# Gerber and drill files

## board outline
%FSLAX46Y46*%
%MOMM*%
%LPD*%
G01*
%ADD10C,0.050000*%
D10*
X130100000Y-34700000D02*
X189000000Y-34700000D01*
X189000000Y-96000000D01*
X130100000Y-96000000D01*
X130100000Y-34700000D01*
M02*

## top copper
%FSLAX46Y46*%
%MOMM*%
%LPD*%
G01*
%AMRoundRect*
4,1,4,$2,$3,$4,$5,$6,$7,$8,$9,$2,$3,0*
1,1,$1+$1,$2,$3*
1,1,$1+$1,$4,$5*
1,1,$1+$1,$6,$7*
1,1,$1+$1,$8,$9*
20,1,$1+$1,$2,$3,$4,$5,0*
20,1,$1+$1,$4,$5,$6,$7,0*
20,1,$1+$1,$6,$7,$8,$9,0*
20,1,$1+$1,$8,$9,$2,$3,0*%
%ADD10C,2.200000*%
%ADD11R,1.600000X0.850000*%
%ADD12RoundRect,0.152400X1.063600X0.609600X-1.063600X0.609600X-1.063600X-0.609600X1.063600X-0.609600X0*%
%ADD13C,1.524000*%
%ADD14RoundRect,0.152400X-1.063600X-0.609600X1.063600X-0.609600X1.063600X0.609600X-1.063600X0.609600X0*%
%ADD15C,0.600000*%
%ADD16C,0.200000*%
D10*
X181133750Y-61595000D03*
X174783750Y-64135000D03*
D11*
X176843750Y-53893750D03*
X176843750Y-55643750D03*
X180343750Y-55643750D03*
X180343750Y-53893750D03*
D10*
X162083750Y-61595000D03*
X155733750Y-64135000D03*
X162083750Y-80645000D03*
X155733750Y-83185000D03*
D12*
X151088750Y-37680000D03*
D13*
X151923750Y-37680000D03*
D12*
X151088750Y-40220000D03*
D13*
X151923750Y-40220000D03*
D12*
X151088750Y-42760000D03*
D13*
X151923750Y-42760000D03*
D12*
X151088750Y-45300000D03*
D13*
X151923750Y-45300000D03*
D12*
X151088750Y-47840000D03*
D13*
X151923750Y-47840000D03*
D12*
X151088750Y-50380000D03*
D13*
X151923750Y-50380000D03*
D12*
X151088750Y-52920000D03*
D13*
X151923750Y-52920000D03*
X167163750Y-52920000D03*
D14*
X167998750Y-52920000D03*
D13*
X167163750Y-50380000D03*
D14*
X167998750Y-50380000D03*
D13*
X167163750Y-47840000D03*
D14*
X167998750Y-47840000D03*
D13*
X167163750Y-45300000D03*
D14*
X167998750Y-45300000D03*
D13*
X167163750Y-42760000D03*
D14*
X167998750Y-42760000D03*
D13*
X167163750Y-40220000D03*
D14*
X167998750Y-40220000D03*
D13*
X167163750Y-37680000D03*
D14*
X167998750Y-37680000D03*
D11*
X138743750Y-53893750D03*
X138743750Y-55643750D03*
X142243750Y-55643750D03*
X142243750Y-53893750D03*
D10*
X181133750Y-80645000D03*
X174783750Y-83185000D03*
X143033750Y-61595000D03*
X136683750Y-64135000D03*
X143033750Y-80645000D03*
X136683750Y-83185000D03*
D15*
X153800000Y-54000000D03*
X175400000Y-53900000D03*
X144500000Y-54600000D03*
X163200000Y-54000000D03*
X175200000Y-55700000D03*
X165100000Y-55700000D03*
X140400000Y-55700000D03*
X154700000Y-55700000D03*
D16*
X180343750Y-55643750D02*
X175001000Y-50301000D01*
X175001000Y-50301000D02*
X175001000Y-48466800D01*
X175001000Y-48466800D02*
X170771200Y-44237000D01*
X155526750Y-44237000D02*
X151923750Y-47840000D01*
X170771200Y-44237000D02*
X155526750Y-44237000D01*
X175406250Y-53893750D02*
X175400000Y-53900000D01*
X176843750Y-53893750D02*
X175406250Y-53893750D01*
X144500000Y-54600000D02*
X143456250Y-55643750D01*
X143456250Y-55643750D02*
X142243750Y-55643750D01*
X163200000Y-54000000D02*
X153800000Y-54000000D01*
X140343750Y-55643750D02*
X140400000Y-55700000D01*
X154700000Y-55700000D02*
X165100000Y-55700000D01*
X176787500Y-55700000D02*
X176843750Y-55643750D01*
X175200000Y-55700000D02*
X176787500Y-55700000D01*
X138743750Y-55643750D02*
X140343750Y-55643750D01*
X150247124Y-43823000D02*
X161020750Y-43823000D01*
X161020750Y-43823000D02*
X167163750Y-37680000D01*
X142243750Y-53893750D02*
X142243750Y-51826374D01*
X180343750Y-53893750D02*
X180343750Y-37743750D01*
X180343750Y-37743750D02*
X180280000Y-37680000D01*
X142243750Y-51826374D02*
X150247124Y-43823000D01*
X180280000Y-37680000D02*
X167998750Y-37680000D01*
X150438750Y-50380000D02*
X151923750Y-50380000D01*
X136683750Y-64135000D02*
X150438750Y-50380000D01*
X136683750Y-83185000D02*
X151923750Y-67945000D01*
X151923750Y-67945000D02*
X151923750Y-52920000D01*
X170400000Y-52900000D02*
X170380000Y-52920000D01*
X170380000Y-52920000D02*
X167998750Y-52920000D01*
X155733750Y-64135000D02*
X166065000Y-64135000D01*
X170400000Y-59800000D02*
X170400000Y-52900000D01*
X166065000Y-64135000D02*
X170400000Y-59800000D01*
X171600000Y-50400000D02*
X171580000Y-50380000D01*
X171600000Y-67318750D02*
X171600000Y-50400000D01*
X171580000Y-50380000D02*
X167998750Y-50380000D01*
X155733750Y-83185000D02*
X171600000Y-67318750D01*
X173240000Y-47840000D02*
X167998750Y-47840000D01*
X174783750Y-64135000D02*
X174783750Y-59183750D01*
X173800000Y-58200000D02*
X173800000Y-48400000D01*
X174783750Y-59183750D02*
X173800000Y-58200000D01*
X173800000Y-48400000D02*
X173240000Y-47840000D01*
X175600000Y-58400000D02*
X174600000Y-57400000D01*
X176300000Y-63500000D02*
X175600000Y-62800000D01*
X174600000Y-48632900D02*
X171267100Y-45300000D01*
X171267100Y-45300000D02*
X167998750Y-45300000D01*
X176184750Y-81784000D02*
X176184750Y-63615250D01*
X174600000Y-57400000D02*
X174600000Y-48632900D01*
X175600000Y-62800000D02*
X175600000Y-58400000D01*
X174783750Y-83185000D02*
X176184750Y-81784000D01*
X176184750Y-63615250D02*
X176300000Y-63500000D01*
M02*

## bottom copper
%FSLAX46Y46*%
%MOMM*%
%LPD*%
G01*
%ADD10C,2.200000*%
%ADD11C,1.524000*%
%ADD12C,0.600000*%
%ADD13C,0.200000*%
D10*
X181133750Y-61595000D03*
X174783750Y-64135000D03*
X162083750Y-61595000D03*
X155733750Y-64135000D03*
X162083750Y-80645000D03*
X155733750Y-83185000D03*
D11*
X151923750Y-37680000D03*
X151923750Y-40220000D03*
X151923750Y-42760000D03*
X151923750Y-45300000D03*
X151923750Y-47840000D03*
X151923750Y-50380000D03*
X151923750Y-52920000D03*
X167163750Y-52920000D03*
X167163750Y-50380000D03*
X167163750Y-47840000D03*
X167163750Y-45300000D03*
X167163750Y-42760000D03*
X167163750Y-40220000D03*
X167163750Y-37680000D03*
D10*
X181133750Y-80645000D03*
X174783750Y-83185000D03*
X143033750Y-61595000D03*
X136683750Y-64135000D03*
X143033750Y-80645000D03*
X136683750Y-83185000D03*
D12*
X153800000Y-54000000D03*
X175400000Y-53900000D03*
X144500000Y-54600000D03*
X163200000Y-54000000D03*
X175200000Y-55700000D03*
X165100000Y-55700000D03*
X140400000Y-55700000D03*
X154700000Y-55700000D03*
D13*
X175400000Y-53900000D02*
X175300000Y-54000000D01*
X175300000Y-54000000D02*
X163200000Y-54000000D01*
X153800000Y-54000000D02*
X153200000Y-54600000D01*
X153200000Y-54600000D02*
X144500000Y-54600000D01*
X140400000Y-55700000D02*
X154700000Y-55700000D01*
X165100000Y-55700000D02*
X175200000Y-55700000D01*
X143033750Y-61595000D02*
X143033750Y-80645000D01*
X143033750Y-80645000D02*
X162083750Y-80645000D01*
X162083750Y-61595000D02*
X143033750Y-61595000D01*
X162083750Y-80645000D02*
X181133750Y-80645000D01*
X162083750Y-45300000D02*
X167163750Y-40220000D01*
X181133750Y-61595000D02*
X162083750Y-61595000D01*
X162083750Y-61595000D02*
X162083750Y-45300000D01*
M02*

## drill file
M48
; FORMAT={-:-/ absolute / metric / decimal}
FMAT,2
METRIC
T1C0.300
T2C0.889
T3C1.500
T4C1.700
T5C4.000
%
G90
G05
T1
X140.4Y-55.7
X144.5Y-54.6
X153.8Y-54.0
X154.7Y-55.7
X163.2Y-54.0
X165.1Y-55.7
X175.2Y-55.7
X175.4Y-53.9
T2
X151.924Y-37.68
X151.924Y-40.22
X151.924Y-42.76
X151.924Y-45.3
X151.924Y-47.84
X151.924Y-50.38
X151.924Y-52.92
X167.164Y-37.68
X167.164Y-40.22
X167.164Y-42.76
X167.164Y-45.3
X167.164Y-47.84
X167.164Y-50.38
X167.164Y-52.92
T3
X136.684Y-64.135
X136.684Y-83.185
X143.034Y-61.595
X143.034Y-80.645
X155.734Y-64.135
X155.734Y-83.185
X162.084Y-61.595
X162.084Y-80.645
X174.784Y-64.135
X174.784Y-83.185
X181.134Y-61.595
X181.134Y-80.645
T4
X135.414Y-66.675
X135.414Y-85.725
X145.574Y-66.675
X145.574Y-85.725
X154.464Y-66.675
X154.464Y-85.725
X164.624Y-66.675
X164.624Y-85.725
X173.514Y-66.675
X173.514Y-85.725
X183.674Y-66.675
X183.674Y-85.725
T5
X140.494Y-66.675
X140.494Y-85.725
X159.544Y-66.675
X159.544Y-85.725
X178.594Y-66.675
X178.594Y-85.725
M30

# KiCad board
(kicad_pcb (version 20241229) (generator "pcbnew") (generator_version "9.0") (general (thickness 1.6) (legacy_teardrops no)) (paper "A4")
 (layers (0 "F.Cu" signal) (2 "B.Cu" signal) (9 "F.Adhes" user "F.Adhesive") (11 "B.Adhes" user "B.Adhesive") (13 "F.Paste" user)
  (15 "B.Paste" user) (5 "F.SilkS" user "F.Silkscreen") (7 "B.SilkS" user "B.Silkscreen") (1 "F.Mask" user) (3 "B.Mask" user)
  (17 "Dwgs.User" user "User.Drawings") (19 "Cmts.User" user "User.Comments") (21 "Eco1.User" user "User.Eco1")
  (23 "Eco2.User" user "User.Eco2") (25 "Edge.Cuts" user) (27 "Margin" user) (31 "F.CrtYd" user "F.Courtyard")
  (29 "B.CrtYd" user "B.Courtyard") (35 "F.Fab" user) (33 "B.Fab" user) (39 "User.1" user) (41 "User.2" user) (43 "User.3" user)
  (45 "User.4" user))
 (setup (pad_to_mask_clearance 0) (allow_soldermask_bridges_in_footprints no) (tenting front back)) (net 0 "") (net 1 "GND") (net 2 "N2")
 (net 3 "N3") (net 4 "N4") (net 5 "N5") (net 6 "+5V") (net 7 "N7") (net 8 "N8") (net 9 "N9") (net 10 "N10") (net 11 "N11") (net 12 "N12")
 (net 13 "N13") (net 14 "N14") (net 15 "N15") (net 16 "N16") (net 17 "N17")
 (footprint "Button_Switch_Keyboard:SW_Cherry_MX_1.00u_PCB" (layer "F.Cu") (at 181.13375 61.595)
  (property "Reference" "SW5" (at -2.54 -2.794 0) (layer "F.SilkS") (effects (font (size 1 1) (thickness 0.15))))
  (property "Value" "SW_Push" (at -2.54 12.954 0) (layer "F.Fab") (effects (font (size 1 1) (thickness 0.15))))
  (pad "" np_thru_hole circle (at -7.62 5.08) (size 1.7 1.7) (drill 1.7) (layers "*.Cu" "*.Mask"))
  (pad "" np_thru_hole circle (at -2.54 5.08) (size 4 4) (drill 4) (layers "*.Cu" "*.Mask"))
  (pad "" np_thru_hole circle (at 2.54 5.08) (size 1.7 1.7) (drill 1.7) (layers "*.Cu" "*.Mask"))
  (pad "1" thru_hole circle (at 0 0) (size 2.2 2.2) (drill 1.5) (layers "*.Cu" "*.Mask") (remove_unused_layers no) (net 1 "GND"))
  (pad "2" thru_hole circle (at -6.35 2.54) (size 2.2 2.2) (drill 1.5) (layers "*.Cu" "*.Mask") (remove_unused_layers no) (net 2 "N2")))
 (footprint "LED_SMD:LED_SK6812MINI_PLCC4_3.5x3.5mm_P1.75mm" (layer "F.Cu") (at 178.59375 54.76875)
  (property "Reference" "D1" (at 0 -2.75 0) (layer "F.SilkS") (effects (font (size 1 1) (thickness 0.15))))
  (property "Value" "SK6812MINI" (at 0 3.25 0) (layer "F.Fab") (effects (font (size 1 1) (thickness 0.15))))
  (pad "1" smd rect (at -1.75 -0.875) (size 1.6 0.85) (layers "F.Cu" "F.Mask" "F.Paste") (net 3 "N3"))
  (pad "2" smd rect (at -1.75 0.875) (size 1.6 0.85) (layers "F.Cu" "F.Mask" "F.Paste") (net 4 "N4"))
  (pad "3" smd rect (at 1.75 0.875) (size 1.6 0.85) (layers "F.Cu" "F.Mask" "F.Paste") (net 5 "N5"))
  (pad "4" smd rect (at 1.75 -0.875) (size 1.6 0.85) (layers "F.Cu" "F.Mask" "F.Paste") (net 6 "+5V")))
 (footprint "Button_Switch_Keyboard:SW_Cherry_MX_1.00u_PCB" (layer "F.Cu") (at 162.08375 61.595)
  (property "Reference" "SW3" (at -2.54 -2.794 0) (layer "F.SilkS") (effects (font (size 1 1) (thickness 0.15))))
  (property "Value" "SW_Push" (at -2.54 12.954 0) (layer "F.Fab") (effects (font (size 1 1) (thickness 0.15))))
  (pad "" np_thru_hole circle (at -7.62 5.08) (size 1.7 1.7) (drill 1.7) (layers "*.Cu" "*.Mask"))
  (pad "" np_thru_hole circle (at -2.54 5.08) (size 4 4) (drill 4) (layers "*.Cu" "*.Mask"))
  (pad "" np_thru_hole circle (at 2.54 5.08) (size 1.7 1.7) (drill 1.7) (layers "*.Cu" "*.Mask"))
  (pad "1" thru_hole circle (at 0 0) (size 2.2 2.2) (drill 1.5) (layers "*.Cu" "*.Mask") (remove_unused_layers no) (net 1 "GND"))
  (pad "2" thru_hole circle (at -6.35 2.54) (size 2.2 2.2) (drill 1.5) (layers "*.Cu" "*.Mask") (remove_unused_layers no) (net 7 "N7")))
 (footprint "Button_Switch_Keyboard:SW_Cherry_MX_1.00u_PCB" (layer "F.Cu") (at 162.08375 80.645)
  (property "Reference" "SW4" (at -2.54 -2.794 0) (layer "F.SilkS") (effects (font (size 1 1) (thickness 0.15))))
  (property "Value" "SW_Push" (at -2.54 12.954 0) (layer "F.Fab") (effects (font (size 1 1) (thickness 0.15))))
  (pad "" np_thru_hole circle (at -7.62 5.08) (size 1.7 1.7) (drill 1.7) (layers "*.Cu" "*.Mask"))
  (pad "" np_thru_hole circle (at -2.54 5.08) (size 4 4) (drill 4) (layers "*.Cu" "*.Mask"))
  (pad "" np_thru_hole circle (at 2.54 5.08) (size 1.7 1.7) (drill 1.7) (layers "*.Cu" "*.Mask"))
  (pad "1" thru_hole circle (at 0 0) (size 2.2 2.2) (drill 1.5) (layers "*.Cu" "*.Mask") (remove_unused_layers no) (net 1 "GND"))
  (pad "2" thru_hole circle (at -6.35 2.54) (size 2.2 2.2) (drill 1.5) (layers "*.Cu" "*.Mask") (remove_unused_layers no) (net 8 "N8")))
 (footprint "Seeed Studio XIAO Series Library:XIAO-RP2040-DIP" (layer "F.Cu") (at 159.54375 45.3)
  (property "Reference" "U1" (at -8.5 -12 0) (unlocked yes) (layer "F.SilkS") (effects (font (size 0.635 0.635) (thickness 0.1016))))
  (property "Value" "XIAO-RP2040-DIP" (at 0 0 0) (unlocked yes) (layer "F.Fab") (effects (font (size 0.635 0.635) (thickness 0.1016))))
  (pad "1" smd roundrect (at -8.455 -7.62 180) (size 2.432 1.524) (layers "F.Cu" "F.Mask") (roundrect_rratio 0.1) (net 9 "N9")
   (thermal_bridge_angle 45))
  (pad "1" thru_hole circle (at -7.62 -7.62 180) (size 1.524 1.524) (drill 0.889) (layers "*.Cu" "*.Mask") (remove_unused_layers no)
   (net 9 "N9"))
  (pad "2" smd roundrect (at -8.455 -5.08 180) (size 2.432 1.524) (layers "F.Cu" "F.Mask") (roundrect_rratio 0.1) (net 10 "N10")
   (thermal_bridge_angle 45))
  (pad "2" thru_hole circle (at -7.62 -5.08 180) (size 1.524 1.524) (drill 0.889) (layers "*.Cu" "*.Mask") (remove_unused_layers no)
   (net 10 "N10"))
  (pad "3" smd roundrect (at -8.455 -2.54 180) (size 2.432 1.524) (layers "F.Cu" "F.Mask") (roundrect_rratio 0.1) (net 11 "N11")
   (thermal_bridge_angle 45))
  (pad "3" thru_hole circle (at -7.62 -2.54 180) (size 1.524 1.524) (drill 0.889) (layers "*.Cu" "*.Mask") (remove_unused_layers no)
   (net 11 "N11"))
  (pad "4" smd roundrect (at -8.455 0 180) (size 2.432 1.524) (layers "F.Cu" "F.Mask") (roundrect_rratio 0.1) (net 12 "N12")
   (thermal_bridge_angle 45))
  (pad "4" thru_hole circle (at -7.62 0 180) (size 1.524 1.524) (drill 0.889) (layers "*.Cu" "*.Mask") (remove_unused_layers no)
   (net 12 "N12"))
  (pad "5" smd roundrect (at -8.455 2.54 180) (size 2.432 1.524) (layers "F.Cu" "F.Mask") (roundrect_rratio 0.1) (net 5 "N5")
   (thermal_bridge_angle 45))
  (pad "5" thru_hole circle (at -7.62 2.54 180) (size 1.524 1.524) (drill 0.889) (layers "*.Cu" "*.Mask") (remove_unused_layers no)
   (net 5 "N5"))
  (pad "6" smd roundrect (at -8.455 5.08 180) (size 2.432 1.524) (layers "F.Cu" "F.Mask") (roundrect_rratio 0.1) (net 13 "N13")
   (thermal_bridge_angle 45))
  (pad "6" thru_hole circle (at -7.62 5.08 180) (size 1.524 1.524) (drill 0.889) (layers "*.Cu" "*.Mask") (remove_unused_layers no)
   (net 13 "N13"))
  (pad "7" smd roundrect (at -8.455 7.62 180) (size 2.432 1.524) (layers "F.Cu" "F.Mask") (roundrect_rratio 0.1) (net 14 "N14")
   (thermal_bridge_angle 45))
  (pad "7" thru_hole circle (at -7.62 7.62 180) (size 1.524 1.524) (drill 0.889) (layers "*.Cu" "*.Mask") (remove_unused_layers no)
   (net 14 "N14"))
  (pad "8" thru_hole circle (at 7.62 7.62) (size 1.524 1.524) (drill 0.889) (layers "*.Cu" "*.Mask") (remove_unused_layers no) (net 7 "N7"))
  (pad "8" smd roundrect (at 8.455 7.62) (size 2.432 1.524) (layers "F.Cu" "F.Mask") (roundrect_rratio 0.1) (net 7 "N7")
   (thermal_bridge_angle 45))
  (pad "9" thru_hole circle (at 7.62 5.08) (size 1.524 1.524) (drill 0.889) (layers "*.Cu" "*.Mask") (remove_unused_layers no) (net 8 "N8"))
  (pad "9" smd roundrect (at 8.455 5.08) (size 2.432 1.524) (layers "F.Cu" "F.Mask") (roundrect_rratio 0.1) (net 8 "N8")
   (thermal_bridge_angle 45))
  (pad "10" thru_hole circle (at 7.62 2.54) (size 1.524 1.524) (drill 0.889) (layers "*.Cu" "*.Mask") (remove_unused_layers no) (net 2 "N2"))
  (pad "10" smd roundrect (at 8.455 2.54) (size 2.432 1.524) (layers "F.Cu" "F.Mask") (roundrect_rratio 0.1) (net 2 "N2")
   (thermal_bridge_angle 45))
  (pad "11" thru_hole circle (at 7.62 0) (size 1.524 1.524) (drill 0.889) (layers "*.Cu" "*.Mask") (remove_unused_layers no) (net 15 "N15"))
  (pad "11" smd roundrect (at 8.455 0) (size 2.432 1.524) (layers "F.Cu" "F.Mask") (roundrect_rratio 0.1) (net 15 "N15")
   (thermal_bridge_angle 45))
  (pad "12" thru_hole circle (at 7.62 -2.54) (size 1.524 1.524) (drill 0.889) (layers "*.Cu" "*.Mask") (remove_unused_layers no)
   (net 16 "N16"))
  (pad "12" smd roundrect (at 8.455 -2.54) (size 2.432 1.524) (layers "F.Cu" "F.Mask") (roundrect_rratio 0.1) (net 16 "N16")
   (thermal_bridge_angle 45))
  (pad "13" thru_hole circle (at 7.62 -5.08) (size 1.524 1.524) (drill 0.889) (layers "*.Cu" "*.Mask") (remove_unused_layers no)
   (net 1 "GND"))
  (pad "13" smd roundrect (at 8.455 -5.08) (size 2.432 1.524) (layers "F.Cu" "F.Mask") (roundrect_rratio 0.1) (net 1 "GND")
   (thermal_bridge_angle 45))
  (pad "14" thru_hole circle (at 7.62 -7.62) (size 1.524 1.524) (drill 0.889) (layers "*.Cu" "*.Mask") (remove_unused_layers no)
   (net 6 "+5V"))
  (pad "14" smd roundrect (at 8.455 -7.62) (size 2.432 1.524) (layers "F.Cu" "F.Mask") (roundrect_rratio 0.1) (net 6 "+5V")
   (thermal_bridge_angle 45)))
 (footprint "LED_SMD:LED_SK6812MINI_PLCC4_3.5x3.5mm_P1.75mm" (layer "F.Cu") (at 140.49375 54.76875)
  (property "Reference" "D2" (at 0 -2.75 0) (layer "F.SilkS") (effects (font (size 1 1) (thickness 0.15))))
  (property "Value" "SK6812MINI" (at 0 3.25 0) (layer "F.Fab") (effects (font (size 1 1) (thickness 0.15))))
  (pad "1" smd rect (at -1.75 -0.875) (size 1.6 0.85) (layers "F.Cu" "F.Mask" "F.Paste") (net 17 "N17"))
  (pad "2" smd rect (at -1.75 0.875) (size 1.6 0.85) (layers "F.Cu" "F.Mask" "F.Paste") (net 4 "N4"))
  (pad "3" smd rect (at 1.75 0.875) (size 1.6 0.85) (layers "F.Cu" "F.Mask" "F.Paste") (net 3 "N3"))
  (pad "4" smd rect (at 1.75 -0.875) (size 1.6 0.85) (layers "F.Cu" "F.Mask" "F.Paste") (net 6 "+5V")))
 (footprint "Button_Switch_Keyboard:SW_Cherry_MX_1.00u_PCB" (layer "F.Cu") (at 181.13375 80.645)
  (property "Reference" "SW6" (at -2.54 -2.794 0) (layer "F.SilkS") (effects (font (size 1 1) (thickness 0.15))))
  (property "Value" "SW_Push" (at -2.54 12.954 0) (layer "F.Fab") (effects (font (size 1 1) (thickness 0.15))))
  (pad "" np_thru_hole circle (at -7.62 5.08) (size 1.7 1.7) (drill 1.7) (layers "*.Cu" "*.Mask"))
  (pad "" np_thru_hole circle (at -2.54 5.08) (size 4 4) (drill 4) (layers "*.Cu" "*.Mask"))
  (pad "" np_thru_hole circle (at 2.54 5.08) (size 1.7 1.7) (drill 1.7) (layers "*.Cu" "*.Mask"))
  (pad "1" thru_hole circle (at 0 0) (size 2.2 2.2) (drill 1.5) (layers "*.Cu" "*.Mask") (remove_unused_layers no) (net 1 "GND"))
  (pad "2" thru_hole circle (at -6.35 2.54) (size 2.2 2.2) (drill 1.5) (layers "*.Cu" "*.Mask") (remove_unused_layers no) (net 15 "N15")))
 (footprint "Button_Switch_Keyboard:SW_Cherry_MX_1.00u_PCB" (layer "F.Cu") (at 143.03375 61.595)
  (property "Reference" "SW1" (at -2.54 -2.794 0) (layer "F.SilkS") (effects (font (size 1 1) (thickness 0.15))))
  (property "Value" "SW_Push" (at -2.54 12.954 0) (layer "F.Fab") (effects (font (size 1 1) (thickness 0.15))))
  (pad "" np_thru_hole circle (at -7.62 5.08) (size 1.7 1.7) (drill 1.7) (layers "*.Cu" "*.Mask"))
  (pad "" np_thru_hole circle (at -2.54 5.08) (size 4 4) (drill 4) (layers "*.Cu" "*.Mask"))
  (pad "" np_thru_hole circle (at 2.54 5.08) (size 1.7 1.7) (drill 1.7) (layers "*.Cu" "*.Mask"))
  (pad "1" thru_hole circle (at 0 0) (size 2.2 2.2) (drill 1.5) (layers "*.Cu" "*.Mask") (remove_unused_layers no) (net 1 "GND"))
  (pad "2" thru_hole circle (at -6.35 2.54) (size 2.2 2.2) (drill 1.5) (layers "*.Cu" "*.Mask") (remove_unused_layers no) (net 13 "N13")))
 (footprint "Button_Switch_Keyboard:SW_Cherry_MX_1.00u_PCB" (layer "F.Cu") (at 143.03375 80.645)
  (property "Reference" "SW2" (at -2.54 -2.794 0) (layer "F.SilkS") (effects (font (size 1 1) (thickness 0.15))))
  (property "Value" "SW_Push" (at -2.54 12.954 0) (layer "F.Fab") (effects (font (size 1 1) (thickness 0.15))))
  (pad "" np_thru_hole circle (at -7.62 5.08) (size 1.7 1.7) (drill 1.7) (layers "*.Cu" "*.Mask"))
  (pad "" np_thru_hole circle (at -2.54 5.08) (size 4 4) (drill 4) (layers "*.Cu" "*.Mask"))
  (pad "" np_thru_hole circle (at 2.54 5.08) (size 1.7 1.7) (drill 1.7) (layers "*.Cu" "*.Mask"))
  (pad "1" thru_hole circle (at 0 0) (size 2.2 2.2) (drill 1.5) (layers "*.Cu" "*.Mask") (remove_unused_layers no) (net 1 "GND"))
  (pad "2" thru_hole circle (at -6.35 2.54) (size 2.2 2.2) (drill 1.5) (layers "*.Cu" "*.Mask") (remove_unused_layers no) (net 14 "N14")))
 (gr_rect (start 130.1 34.7) (end 189 96) (stroke (width 0.05) (type default)) (fill no) (layer "Edge.Cuts"))
 (segment (start 180.34375 55.64375) (end 175.001 50.301) (width 0.2) (layer "F.Cu") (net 5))
 (segment (start 175.001 50.301) (end 175.001 48.4668) (width 0.2) (layer "F.Cu") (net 5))
 (segment (start 175.001 48.4668) (end 170.7712 44.237) (width 0.2) (layer "F.Cu") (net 5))
 (segment (start 155.52675 44.237) (end 151.92375 47.84) (width 0.2) (layer "F.Cu") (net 5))
 (segment (start 170.7712 44.237) (end 155.52675 44.237) (width 0.2) (layer "F.Cu") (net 5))
 (segment (start 175.40625 53.89375) (end 175.4 53.9) (width 0.2) (layer "F.Cu") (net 3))
 (segment (start 176.84375 53.89375) (end 175.40625 53.89375) (width 0.2) (layer "F.Cu") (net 3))
 (segment (start 144.5 54.6) (end 143.45625 55.64375) (width 0.2) (layer "F.Cu") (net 3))
 (segment (start 143.45625 55.64375) (end 142.24375 55.64375) (width 0.2) (layer "F.Cu") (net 3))
 (segment (start 163.2 54) (end 153.8 54) (width 0.2) (layer "F.Cu") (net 3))
 (via (at 153.8 54) (size 0.6) (drill 0.3) (layers "F.Cu" "B.Cu") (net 3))
 (via (at 175.4 53.9) (size 0.6) (drill 0.3) (layers "F.Cu" "B.Cu") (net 3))
 (via (at 144.5 54.6) (size 0.6) (drill 0.3) (layers "F.Cu" "B.Cu") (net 3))
 (via (at 163.2 54) (size 0.6) (drill 0.3) (layers "F.Cu" "B.Cu") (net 3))
 (segment (start 175.4 53.9) (end 175.3 54) (width 0.2) (layer "B.Cu") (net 3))
 (segment (start 175.3 54) (end 163.2 54) (width 0.2) (layer "B.Cu") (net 3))
 (segment (start 153.8 54) (end 153.2 54.6) (width 0.2) (layer "B.Cu") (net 3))
 (segment (start 153.2 54.6) (end 144.5 54.6) (width 0.2) (layer "B.Cu") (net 3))
 (segment (start 140.34375 55.64375) (end 140.4 55.7) (width 0.2) (layer "F.Cu") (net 4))
 (segment (start 154.7 55.7) (end 165.1 55.7) (width 0.2) (layer "F.Cu") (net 4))
 (segment (start 176.7875 55.7) (end 176.84375 55.64375) (width 0.2) (layer "F.Cu") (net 4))
 (segment (start 175.2 55.7) (end 176.7875 55.7) (width 0.2) (layer "F.Cu") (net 4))
 (segment (start 138.74375 55.64375) (end 140.34375 55.64375) (width 0.2) (layer "F.Cu") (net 4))
 (via (at 175.2 55.7) (size 0.6) (drill 0.3) (layers "F.Cu" "B.Cu") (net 4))
 (via (at 165.1 55.7) (size 0.6) (drill 0.3) (layers "F.Cu" "B.Cu") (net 4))
 (via (at 140.4 55.7) (size 0.6) (drill 0.3) (layers "F.Cu" "B.Cu") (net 4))
 (via (at 154.7 55.7) (size 0.6) (drill 0.3) (layers "F.Cu" "B.Cu") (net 4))
 (segment (start 140.4 55.7) (end 154.7 55.7) (width 0.2) (layer "B.Cu") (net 4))
 (segment (start 165.1 55.7) (end 175.2 55.7) (width 0.2) (layer "B.Cu") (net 4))
 (segment (start 150.247124 43.823) (end 161.02075 43.823) (width 0.2) (layer "F.Cu") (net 6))
 (segment (start 161.02075 43.823) (end 167.16375 37.68) (width 0.2) (layer "F.Cu") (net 6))
 (segment (start 142.24375 53.89375) (end 142.24375 51.826374) (width 0.2) (layer "F.Cu") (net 6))
 (segment (start 180.34375 53.89375) (end 180.34375 37.74375) (width 0.2) (layer "F.Cu") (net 6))
 (segment (start 180.34375 37.74375) (end 180.28 37.68) (width 0.2) (layer "F.Cu") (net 6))
 (segment (start 142.24375 51.826374) (end 150.247124 43.823) (width 0.2) (layer "F.Cu") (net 6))
 (segment (start 180.28 37.68) (end 167.99875 37.68) (width 0.2) (layer "F.Cu") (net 6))
 (segment (start 143.03375 61.595) (end 143.03375 80.645) (width 0.2) (layer "B.Cu") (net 1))
 (segment (start 143.03375 80.645) (end 162.08375 80.645) (width 0.2) (layer "B.Cu") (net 1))
 (segment (start 162.08375 61.595) (end 143.03375 61.595) (width 0.2) (layer "B.Cu") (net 1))
 (segment (start 162.08375 80.645) (end 181.13375 80.645) (width 0.2) (layer "B.Cu") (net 1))
 (segment (start 162.08375 45.3) (end 167.16375 40.22) (width 0.2) (layer "B.Cu") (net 1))
 (segment (start 181.13375 61.595) (end 162.08375 61.595) (width 0.2) (layer "B.Cu") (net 1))
 (segment (start 162.08375 61.595) (end 162.08375 45.3) (width 0.2) (layer "B.Cu") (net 1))
 (segment (start 150.43875 50.38) (end 151.92375 50.38) (width 0.2) (layer "F.Cu") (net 13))
 (segment (start 136.68375 64.135) (end 150.43875 50.38) (width 0.2) (layer "F.Cu") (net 13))
 (segment (start 136.68375 83.185) (end 151.92375 67.945) (width 0.2) (layer "F.Cu") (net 14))
 (segment (start 151.92375 67.945) (end 151.92375 52.92) (width 0.2) (layer "F.Cu") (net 14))
 (segment (start 170.4 52.9) (end 170.38 52.92) (width 0.2) (layer "F.Cu") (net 7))
 (segment (start 170.38 52.92) (end 167.99875 52.92) (width 0.2) (layer "F.Cu") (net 7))
 (segment (start 155.73375 64.135) (end 166.065 64.135) (width 0.2) (layer "F.Cu") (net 7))
 (segment (start 170.4 59.8) (end 170.4 52.9) (width 0.2) (layer "F.Cu") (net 7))
 (segment (start 166.065 64.135) (end 170.4 59.8) (width 0.2) (layer "F.Cu") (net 7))
 (segment (start 171.6 50.4) (end 171.58 50.38) (width 0.2) (layer "F.Cu") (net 8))
 (segment (start 171.6 67.31875) (end 171.6 50.4) (width 0.2) (layer "F.Cu") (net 8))
 (segment (start 171.58 50.38) (end 167.99875 50.38) (width 0.2) (layer "F.Cu") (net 8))
 (segment (start 155.73375 83.185) (end 171.6 67.31875) (width 0.2) (layer "F.Cu") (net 8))
 (segment (start 173.24 47.84) (end 167.99875 47.84) (width 0.2) (layer "F.Cu") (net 2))
 (segment (start 174.78375 64.135) (end 174.78375 59.18375) (width 0.2) (layer "F.Cu") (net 2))
 (segment (start 173.8 58.2) (end 173.8 48.4) (width 0.2) (layer "F.Cu") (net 2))
 (segment (start 174.78375 59.18375) (end 173.8 58.2) (width 0.2) (layer "F.Cu") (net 2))
 (segment (start 173.8 48.4) (end 173.24 47.84) (width 0.2) (layer "F.Cu") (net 2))
 (segment (start 175.6 58.4) (end 174.6 57.4) (width 0.2) (layer "F.Cu") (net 15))
 (segment (start 176.3 63.5) (end 175.6 62.8) (width 0.2) (layer "F.Cu") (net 15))
 (segment (start 174.6 48.6329) (end 171.2671 45.3) (width 0.2) (layer "F.Cu") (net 15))
 (segment (start 171.2671 45.3) (end 167.99875 45.3) (width 0.2) (layer "F.Cu") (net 15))
 (segment (start 176.18475 81.784) (end 176.18475 63.61525) (width 0.2) (layer "F.Cu") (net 15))
 (segment (start 174.6 57.4) (end 174.6 48.6329) (width 0.2) (layer "F.Cu") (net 15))
 (segment (start 175.6 62.8) (end 175.6 58.4) (width 0.2) (layer "F.Cu") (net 15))
 (segment (start 174.78375 83.185) (end 176.18475 81.784) (width 0.2) (layer "F.Cu") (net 15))
 (segment (start 176.18475 63.61525) (end 176.3 63.5) (width 0.2) (layer "F.Cu") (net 15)))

